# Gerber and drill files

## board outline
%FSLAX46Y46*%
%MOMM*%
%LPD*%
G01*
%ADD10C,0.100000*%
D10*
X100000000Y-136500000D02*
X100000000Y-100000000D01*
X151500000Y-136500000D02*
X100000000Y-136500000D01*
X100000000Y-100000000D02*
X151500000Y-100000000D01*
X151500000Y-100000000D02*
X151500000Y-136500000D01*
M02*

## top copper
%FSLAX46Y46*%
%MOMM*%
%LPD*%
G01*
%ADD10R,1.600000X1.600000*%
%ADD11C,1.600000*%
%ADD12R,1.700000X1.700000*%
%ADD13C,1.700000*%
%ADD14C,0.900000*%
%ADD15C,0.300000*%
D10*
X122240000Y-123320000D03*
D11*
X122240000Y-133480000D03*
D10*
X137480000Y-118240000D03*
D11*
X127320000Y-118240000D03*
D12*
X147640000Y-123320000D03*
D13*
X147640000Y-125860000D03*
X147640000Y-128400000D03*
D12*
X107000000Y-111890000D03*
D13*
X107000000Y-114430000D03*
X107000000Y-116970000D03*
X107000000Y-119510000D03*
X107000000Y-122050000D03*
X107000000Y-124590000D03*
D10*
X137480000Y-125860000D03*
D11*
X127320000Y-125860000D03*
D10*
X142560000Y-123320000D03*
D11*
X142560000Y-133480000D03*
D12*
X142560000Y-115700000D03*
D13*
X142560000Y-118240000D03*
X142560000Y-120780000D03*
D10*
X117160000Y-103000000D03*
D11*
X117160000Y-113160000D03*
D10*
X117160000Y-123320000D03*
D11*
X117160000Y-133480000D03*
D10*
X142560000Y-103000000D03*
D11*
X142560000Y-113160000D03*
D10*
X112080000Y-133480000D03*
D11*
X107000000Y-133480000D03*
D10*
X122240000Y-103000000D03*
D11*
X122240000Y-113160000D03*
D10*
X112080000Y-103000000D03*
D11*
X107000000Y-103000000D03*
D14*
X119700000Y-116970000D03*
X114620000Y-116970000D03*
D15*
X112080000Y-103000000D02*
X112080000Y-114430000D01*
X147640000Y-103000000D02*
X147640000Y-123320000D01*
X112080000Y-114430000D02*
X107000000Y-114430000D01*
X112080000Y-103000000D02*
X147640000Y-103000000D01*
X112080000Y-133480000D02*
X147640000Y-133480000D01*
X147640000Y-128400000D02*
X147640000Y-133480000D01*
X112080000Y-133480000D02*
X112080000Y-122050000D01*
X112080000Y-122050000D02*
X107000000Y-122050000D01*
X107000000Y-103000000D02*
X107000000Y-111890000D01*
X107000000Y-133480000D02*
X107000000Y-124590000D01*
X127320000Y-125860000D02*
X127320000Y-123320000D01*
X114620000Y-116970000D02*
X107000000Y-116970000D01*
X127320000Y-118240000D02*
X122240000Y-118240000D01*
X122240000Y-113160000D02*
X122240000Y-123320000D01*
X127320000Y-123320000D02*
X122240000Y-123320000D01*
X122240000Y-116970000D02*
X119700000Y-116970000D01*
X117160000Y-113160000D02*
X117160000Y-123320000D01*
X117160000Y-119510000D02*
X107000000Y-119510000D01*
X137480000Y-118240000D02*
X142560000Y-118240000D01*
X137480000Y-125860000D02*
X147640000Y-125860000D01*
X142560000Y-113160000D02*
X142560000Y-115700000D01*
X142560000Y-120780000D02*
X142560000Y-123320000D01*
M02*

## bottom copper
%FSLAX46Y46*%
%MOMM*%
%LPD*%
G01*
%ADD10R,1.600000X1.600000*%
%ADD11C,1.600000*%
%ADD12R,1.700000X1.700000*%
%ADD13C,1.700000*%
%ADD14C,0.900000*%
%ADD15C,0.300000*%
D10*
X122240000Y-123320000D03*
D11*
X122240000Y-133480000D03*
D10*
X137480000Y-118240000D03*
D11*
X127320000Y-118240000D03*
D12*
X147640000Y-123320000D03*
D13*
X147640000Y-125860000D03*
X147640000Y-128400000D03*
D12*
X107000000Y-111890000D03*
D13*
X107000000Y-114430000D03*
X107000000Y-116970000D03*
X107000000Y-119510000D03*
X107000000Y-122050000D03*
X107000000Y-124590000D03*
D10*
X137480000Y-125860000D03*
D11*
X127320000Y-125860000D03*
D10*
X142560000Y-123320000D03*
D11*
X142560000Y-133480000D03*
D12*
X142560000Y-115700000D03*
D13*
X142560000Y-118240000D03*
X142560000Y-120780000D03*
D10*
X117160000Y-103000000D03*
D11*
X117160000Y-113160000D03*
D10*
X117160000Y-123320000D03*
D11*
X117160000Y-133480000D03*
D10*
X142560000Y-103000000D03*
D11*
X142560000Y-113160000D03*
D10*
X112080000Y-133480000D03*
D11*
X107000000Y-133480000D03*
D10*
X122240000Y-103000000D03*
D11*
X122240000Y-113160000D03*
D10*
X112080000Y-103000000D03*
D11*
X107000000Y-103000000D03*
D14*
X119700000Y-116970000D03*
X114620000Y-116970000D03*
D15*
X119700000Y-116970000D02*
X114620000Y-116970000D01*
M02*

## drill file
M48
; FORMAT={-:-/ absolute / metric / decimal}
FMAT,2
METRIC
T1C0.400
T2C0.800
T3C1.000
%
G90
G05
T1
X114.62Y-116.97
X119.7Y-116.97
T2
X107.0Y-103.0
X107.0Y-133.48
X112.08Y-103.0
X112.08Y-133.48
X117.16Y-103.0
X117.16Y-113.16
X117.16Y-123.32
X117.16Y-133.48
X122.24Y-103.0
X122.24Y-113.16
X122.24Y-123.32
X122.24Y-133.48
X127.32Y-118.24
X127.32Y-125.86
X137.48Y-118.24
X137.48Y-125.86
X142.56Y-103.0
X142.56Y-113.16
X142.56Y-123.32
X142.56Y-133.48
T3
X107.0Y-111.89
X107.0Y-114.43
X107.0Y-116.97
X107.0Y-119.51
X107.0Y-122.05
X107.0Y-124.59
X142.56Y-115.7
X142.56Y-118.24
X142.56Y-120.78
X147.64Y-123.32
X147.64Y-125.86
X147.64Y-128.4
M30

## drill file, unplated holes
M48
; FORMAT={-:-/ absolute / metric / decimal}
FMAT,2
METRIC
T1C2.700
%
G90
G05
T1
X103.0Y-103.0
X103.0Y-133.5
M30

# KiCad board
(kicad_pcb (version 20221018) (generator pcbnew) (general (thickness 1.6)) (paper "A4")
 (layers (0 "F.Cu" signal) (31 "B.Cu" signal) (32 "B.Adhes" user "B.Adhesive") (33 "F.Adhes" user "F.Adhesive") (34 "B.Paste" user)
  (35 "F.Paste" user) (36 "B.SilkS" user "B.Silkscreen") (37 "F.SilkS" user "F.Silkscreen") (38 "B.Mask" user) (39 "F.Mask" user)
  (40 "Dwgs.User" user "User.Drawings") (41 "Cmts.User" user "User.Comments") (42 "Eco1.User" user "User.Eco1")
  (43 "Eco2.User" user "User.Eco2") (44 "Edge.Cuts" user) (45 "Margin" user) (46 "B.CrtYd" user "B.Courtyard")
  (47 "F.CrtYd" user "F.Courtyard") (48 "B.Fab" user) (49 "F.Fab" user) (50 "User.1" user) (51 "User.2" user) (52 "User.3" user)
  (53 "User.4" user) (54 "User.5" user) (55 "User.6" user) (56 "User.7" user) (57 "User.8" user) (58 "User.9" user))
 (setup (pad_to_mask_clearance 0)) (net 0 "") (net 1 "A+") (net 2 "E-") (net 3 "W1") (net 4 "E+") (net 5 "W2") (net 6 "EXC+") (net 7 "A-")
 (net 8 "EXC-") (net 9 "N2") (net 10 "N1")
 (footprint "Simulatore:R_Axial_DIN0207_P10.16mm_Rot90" (layer "F.Cu") (at 122.24 123.32)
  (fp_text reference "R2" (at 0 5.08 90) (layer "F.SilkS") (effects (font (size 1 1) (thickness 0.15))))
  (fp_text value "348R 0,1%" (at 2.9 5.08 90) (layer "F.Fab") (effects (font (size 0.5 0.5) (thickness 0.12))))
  (pad "1" thru_hole rect (at 0 0) (size 1.6 1.6) (drill 0.8) (layers "*.Cu" "*.Mask") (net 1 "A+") (thermal_bridge_angle 45))
  (pad "2" thru_hole circle (at 0 10.16) (size 1.6 1.6) (drill 0.8) (layers "*.Cu" "*.Mask") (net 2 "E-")))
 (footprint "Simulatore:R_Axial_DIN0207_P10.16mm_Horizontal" (layer "F.Cu") (at 132.4 118.24)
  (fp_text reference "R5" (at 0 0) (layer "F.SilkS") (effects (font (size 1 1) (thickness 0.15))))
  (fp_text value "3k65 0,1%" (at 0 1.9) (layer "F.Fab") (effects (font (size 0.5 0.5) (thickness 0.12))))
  (pad "1" thru_hole rect (at 5.08 0) (size 1.6 1.6) (drill 0.8) (layers "*.Cu" "*.Mask") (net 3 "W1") (thermal_bridge_angle 45))
  (pad "2" thru_hole circle (at -5.08 0) (size 1.6 1.6) (drill 0.8) (layers "*.Cu" "*.Mask") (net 1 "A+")))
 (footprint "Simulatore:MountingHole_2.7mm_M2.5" (layer "F.Cu") (at 103 103)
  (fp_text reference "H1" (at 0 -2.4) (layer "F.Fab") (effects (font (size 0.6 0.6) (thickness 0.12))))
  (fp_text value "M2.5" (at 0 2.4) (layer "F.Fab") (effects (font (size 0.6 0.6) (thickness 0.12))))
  (pad "" np_thru_hole circle (at 0 0) (size 2.7 2.7) (drill 2.7) (layers "*.Cu" "*.Mask")))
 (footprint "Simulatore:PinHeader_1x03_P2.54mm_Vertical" (layer "F.Cu") (at 147.64 123.32)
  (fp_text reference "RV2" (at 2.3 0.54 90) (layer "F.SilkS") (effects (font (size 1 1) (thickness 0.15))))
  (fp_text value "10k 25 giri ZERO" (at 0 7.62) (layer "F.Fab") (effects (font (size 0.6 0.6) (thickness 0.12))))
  (pad "1" thru_hole rect (at 0 0) (size 1.7 1.7) (drill 1) (layers "*.Cu" "*.Mask") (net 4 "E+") (thermal_bridge_angle 45))
  (pad "2" thru_hole circle (at 0 2.54) (size 1.7 1.7) (drill 1) (layers "*.Cu" "*.Mask") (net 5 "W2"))
  (pad "3" thru_hole circle (at 0 5.08) (size 1.7 1.7) (drill 1) (layers "*.Cu" "*.Mask") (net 2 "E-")))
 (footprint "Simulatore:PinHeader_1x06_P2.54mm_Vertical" (layer "F.Cu") (at 107 111.89)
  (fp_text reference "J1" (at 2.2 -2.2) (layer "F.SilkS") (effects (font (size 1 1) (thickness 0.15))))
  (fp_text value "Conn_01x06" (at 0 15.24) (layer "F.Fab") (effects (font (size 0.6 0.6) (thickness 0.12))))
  (pad "1" thru_hole rect (at 0 0) (size 1.7 1.7) (drill 1) (layers "*.Cu" "*.Mask") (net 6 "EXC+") (thermal_bridge_angle 45))
  (pad "2" thru_hole circle (at 0 2.54) (size 1.7 1.7) (drill 1) (layers "*.Cu" "*.Mask") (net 4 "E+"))
  (pad "3" thru_hole circle (at 0 5.08) (size 1.7 1.7) (drill 1) (layers "*.Cu" "*.Mask") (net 1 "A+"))
  (pad "4" thru_hole circle (at 0 7.62) (size 1.7 1.7) (drill 1) (layers "*.Cu" "*.Mask") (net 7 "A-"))
  (pad "5" thru_hole circle (at 0 10.16) (size 1.7 1.7) (drill 1) (layers "*.Cu" "*.Mask") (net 2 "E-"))
  (pad "6" thru_hole circle (at 0 12.7) (size 1.7 1.7) (drill 1) (layers "*.Cu" "*.Mask") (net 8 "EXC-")))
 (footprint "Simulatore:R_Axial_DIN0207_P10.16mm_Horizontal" (layer "F.Cu") (at 132.4 125.86)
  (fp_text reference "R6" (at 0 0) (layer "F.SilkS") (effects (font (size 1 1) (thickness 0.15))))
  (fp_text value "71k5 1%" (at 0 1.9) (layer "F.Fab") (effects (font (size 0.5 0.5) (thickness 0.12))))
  (pad "1" thru_hole rect (at 5.08 0) (size 1.6 1.6) (drill 0.8) (layers "*.Cu" "*.Mask") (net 5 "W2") (thermal_bridge_angle 45))
  (pad "2" thru_hole circle (at -5.08 0) (size 1.6 1.6) (drill 0.8) (layers "*.Cu" "*.Mask") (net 1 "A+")))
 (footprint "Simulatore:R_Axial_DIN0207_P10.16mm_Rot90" (layer "F.Cu") (at 142.56 123.32)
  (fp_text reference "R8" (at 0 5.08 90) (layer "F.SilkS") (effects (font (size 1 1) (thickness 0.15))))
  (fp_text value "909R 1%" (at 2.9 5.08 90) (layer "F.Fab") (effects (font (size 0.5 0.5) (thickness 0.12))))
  (pad "1" thru_hole rect (at 0 0) (size 1.6 1.6) (drill 0.8) (layers "*.Cu" "*.Mask") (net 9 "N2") (thermal_bridge_angle 45))
  (pad "2" thru_hole circle (at 0 10.16) (size 1.6 1.6) (drill 0.8) (layers "*.Cu" "*.Mask") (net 2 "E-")))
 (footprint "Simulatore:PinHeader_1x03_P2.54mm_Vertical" (layer "F.Cu") (at 142.56 115.7)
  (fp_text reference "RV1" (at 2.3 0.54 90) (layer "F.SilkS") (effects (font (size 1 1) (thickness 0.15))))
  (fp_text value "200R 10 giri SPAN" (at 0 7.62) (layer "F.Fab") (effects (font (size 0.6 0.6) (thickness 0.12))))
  (pad "1" thru_hole rect (at 0 0) (size 1.7 1.7) (drill 1) (layers "*.Cu" "*.Mask") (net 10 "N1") (thermal_bridge_angle 45))
  (pad "2" thru_hole circle (at 0 2.54) (size 1.7 1.7) (drill 1) (layers "*.Cu" "*.Mask") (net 3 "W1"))
  (pad "3" thru_hole circle (at 0 5.08) (size 1.7 1.7) (drill 1) (layers "*.Cu" "*.Mask") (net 9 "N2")))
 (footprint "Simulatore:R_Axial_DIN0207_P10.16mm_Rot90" (layer "F.Cu") (at 117.16 103)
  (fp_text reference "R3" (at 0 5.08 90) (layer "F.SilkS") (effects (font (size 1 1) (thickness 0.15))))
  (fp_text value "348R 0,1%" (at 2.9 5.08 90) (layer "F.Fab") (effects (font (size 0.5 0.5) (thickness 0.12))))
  (pad "1" thru_hole rect (at 0 0) (size 1.6 1.6) (drill 0.8) (layers "*.Cu" "*.Mask") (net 4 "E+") (thermal_bridge_angle 45))
  (pad "2" thru_hole circle (at 0 10.16) (size 1.6 1.6) (drill 0.8) (layers "*.Cu" "*.Mask") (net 7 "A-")))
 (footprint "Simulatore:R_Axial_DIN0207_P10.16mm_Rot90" (layer "F.Cu") (at 117.16 123.32)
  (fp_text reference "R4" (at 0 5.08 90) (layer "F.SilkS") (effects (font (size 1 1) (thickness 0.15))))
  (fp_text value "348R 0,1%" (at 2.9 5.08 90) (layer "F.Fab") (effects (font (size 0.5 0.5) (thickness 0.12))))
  (pad "1" thru_hole rect (at 0 0) (size 1.6 1.6) (drill 0.8) (layers "*.Cu" "*.Mask") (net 7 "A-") (thermal_bridge_angle 45))
  (pad "2" thru_hole circle (at 0 10.16) (size 1.6 1.6) (drill 0.8) (layers "*.Cu" "*.Mask") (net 2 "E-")))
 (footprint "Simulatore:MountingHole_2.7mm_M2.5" (layer "F.Cu") (at 103 133.5)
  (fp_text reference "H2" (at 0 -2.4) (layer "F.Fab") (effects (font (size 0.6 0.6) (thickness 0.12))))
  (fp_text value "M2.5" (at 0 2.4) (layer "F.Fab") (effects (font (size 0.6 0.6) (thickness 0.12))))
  (pad "" np_thru_hole circle (at 0 0) (size 2.7 2.7) (drill 2.7) (layers "*.Cu" "*.Mask")))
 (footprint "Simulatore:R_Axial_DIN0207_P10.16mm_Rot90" (layer "F.Cu") (at 142.56 103)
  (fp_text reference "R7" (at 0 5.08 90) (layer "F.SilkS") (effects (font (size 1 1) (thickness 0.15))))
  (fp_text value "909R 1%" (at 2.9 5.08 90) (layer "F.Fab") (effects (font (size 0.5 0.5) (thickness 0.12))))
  (pad "1" thru_hole rect (at 0 0) (size 1.6 1.6) (drill 0.8) (layers "*.Cu" "*.Mask") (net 4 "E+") (thermal_bridge_angle 45))
  (pad "2" thru_hole circle (at 0 10.16) (size 1.6 1.6) (drill 0.8) (layers "*.Cu" "*.Mask") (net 10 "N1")))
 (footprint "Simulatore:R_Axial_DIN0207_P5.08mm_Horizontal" (layer "F.Cu") (at 112.08 133.48)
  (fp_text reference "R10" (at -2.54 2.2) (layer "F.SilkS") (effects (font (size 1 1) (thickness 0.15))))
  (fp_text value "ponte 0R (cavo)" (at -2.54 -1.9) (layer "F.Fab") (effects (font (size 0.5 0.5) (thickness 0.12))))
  (pad "1" thru_hole rect (at 0 0) (size 1.6 1.6) (drill 0.8) (layers "*.Cu" "*.Mask") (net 2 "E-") (thermal_bridge_angle 45))
  (pad "2" thru_hole circle (at -5.08 0) (size 1.6 1.6) (drill 0.8) (layers "*.Cu" "*.Mask") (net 8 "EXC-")))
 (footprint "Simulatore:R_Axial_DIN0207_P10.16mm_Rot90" (layer "F.Cu") (at 122.24 103)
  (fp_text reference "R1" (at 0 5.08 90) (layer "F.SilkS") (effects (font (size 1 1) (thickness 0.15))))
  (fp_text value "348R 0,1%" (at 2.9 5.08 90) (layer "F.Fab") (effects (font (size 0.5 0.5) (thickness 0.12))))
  (pad "1" thru_hole rect (at 0 0) (size 1.6 1.6) (drill 0.8) (layers "*.Cu" "*.Mask") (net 4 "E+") (thermal_bridge_angle 45))
  (pad "2" thru_hole circle (at 0 10.16) (size 1.6 1.6) (drill 0.8) (layers "*.Cu" "*.Mask") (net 1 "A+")))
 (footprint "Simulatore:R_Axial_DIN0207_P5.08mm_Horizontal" (layer "F.Cu") (at 112.08 103)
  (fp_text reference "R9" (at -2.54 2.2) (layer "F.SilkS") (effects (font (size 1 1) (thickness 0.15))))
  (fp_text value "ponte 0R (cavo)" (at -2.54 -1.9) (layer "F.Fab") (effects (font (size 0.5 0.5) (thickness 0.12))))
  (pad "1" thru_hole rect (at 0 0) (size 1.6 1.6) (drill 0.8) (layers "*.Cu" "*.Mask") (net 4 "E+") (thermal_bridge_angle 45))
  (pad "2" thru_hole circle (at -5.08 0) (size 1.6 1.6) (drill 0.8) (layers "*.Cu" "*.Mask") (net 6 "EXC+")))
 (gr_line (start 100 136.5) (end 100 100) (stroke (width 0.1) (type default)) (layer "Edge.Cuts"))
 (gr_line (start 151.5 136.5) (end 100 136.5) (stroke (width 0.1) (type default)) (layer "Edge.Cuts"))
 (gr_line (start 100 100) (end 151.5 100) (stroke (width 0.1) (type default)) (layer "Edge.Cuts"))
 (gr_line (start 151.5 100) (end 151.5 136.5) (stroke (width 0.1) (type default)) (layer "Edge.Cuts"))
 (segment (start 112.08 103) (end 112.08 114.43) (width 0.3) (layer "F.Cu") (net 4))
 (segment (start 147.64 103) (end 147.64 123.32) (width 0.3) (layer "F.Cu") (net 4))
 (segment (start 112.08 114.43) (end 107 114.43) (width 0.3) (layer "F.Cu") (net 4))
 (segment (start 112.08 103) (end 147.64 103) (width 0.3) (layer "F.Cu") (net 4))
 (segment (start 112.08 133.48) (end 147.64 133.48) (width 0.3) (layer "F.Cu") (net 2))
 (segment (start 147.64 128.4) (end 147.64 133.48) (width 0.3) (layer "F.Cu") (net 2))
 (segment (start 112.08 133.48) (end 112.08 122.05) (width 0.3) (layer "F.Cu") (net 2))
 (segment (start 112.08 122.05) (end 107 122.05) (width 0.3) (layer "F.Cu") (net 2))
 (segment (start 107 103) (end 107 111.89) (width 0.3) (layer "F.Cu") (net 6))
 (segment (start 107 133.48) (end 107 124.59) (width 0.3) (layer "F.Cu") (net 8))
 (segment (start 127.32 125.86) (end 127.32 123.32) (width 0.3) (layer "F.Cu") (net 1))
 (segment (start 114.62 116.97) (end 107 116.97) (width 0.3) (layer "F.Cu") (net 1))
 (segment (start 127.32 118.24) (end 122.24 118.24) (width 0.3) (layer "F.Cu") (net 1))
 (segment (start 122.24 113.16) (end 122.24 123.32) (width 0.3) (layer "F.Cu") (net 1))
 (segment (start 127.32 123.32) (end 122.24 123.32) (width 0.3) (layer "F.Cu") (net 1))
 (segment (start 122.24 116.97) (end 119.7 116.97) (width 0.3) (layer "F.Cu") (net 1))
 (via (at 119.7 116.97) (size 0.9) (drill 0.4) (layers "F.Cu" "B.Cu") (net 1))
 (via (at 114.62 116.97) (size 0.9) (drill 0.4) (layers "F.Cu" "B.Cu") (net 1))
 (segment (start 119.7 116.97) (end 114.62 116.97) (width 0.3) (layer "B.Cu") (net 1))
 (segment (start 117.16 113.16) (end 117.16 123.32) (width 0.3) (layer "F.Cu") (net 7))
 (segment (start 117.16 119.51) (end 107 119.51) (width 0.3) (layer "F.Cu") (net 7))
 (segment (start 137.48 118.24) (end 142.56 118.24) (width 0.3) (layer "F.Cu") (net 3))
 (segment (start 137.48 125.86) (end 147.64 125.86) (width 0.3) (layer "F.Cu") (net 5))
 (segment (start 142.56 113.16) (end 142.56 115.7) (width 0.3) (layer "F.Cu") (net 10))
 (segment (start 142.56 120.78) (end 142.56 123.32) (width 0.3) (layer "F.Cu") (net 9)))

